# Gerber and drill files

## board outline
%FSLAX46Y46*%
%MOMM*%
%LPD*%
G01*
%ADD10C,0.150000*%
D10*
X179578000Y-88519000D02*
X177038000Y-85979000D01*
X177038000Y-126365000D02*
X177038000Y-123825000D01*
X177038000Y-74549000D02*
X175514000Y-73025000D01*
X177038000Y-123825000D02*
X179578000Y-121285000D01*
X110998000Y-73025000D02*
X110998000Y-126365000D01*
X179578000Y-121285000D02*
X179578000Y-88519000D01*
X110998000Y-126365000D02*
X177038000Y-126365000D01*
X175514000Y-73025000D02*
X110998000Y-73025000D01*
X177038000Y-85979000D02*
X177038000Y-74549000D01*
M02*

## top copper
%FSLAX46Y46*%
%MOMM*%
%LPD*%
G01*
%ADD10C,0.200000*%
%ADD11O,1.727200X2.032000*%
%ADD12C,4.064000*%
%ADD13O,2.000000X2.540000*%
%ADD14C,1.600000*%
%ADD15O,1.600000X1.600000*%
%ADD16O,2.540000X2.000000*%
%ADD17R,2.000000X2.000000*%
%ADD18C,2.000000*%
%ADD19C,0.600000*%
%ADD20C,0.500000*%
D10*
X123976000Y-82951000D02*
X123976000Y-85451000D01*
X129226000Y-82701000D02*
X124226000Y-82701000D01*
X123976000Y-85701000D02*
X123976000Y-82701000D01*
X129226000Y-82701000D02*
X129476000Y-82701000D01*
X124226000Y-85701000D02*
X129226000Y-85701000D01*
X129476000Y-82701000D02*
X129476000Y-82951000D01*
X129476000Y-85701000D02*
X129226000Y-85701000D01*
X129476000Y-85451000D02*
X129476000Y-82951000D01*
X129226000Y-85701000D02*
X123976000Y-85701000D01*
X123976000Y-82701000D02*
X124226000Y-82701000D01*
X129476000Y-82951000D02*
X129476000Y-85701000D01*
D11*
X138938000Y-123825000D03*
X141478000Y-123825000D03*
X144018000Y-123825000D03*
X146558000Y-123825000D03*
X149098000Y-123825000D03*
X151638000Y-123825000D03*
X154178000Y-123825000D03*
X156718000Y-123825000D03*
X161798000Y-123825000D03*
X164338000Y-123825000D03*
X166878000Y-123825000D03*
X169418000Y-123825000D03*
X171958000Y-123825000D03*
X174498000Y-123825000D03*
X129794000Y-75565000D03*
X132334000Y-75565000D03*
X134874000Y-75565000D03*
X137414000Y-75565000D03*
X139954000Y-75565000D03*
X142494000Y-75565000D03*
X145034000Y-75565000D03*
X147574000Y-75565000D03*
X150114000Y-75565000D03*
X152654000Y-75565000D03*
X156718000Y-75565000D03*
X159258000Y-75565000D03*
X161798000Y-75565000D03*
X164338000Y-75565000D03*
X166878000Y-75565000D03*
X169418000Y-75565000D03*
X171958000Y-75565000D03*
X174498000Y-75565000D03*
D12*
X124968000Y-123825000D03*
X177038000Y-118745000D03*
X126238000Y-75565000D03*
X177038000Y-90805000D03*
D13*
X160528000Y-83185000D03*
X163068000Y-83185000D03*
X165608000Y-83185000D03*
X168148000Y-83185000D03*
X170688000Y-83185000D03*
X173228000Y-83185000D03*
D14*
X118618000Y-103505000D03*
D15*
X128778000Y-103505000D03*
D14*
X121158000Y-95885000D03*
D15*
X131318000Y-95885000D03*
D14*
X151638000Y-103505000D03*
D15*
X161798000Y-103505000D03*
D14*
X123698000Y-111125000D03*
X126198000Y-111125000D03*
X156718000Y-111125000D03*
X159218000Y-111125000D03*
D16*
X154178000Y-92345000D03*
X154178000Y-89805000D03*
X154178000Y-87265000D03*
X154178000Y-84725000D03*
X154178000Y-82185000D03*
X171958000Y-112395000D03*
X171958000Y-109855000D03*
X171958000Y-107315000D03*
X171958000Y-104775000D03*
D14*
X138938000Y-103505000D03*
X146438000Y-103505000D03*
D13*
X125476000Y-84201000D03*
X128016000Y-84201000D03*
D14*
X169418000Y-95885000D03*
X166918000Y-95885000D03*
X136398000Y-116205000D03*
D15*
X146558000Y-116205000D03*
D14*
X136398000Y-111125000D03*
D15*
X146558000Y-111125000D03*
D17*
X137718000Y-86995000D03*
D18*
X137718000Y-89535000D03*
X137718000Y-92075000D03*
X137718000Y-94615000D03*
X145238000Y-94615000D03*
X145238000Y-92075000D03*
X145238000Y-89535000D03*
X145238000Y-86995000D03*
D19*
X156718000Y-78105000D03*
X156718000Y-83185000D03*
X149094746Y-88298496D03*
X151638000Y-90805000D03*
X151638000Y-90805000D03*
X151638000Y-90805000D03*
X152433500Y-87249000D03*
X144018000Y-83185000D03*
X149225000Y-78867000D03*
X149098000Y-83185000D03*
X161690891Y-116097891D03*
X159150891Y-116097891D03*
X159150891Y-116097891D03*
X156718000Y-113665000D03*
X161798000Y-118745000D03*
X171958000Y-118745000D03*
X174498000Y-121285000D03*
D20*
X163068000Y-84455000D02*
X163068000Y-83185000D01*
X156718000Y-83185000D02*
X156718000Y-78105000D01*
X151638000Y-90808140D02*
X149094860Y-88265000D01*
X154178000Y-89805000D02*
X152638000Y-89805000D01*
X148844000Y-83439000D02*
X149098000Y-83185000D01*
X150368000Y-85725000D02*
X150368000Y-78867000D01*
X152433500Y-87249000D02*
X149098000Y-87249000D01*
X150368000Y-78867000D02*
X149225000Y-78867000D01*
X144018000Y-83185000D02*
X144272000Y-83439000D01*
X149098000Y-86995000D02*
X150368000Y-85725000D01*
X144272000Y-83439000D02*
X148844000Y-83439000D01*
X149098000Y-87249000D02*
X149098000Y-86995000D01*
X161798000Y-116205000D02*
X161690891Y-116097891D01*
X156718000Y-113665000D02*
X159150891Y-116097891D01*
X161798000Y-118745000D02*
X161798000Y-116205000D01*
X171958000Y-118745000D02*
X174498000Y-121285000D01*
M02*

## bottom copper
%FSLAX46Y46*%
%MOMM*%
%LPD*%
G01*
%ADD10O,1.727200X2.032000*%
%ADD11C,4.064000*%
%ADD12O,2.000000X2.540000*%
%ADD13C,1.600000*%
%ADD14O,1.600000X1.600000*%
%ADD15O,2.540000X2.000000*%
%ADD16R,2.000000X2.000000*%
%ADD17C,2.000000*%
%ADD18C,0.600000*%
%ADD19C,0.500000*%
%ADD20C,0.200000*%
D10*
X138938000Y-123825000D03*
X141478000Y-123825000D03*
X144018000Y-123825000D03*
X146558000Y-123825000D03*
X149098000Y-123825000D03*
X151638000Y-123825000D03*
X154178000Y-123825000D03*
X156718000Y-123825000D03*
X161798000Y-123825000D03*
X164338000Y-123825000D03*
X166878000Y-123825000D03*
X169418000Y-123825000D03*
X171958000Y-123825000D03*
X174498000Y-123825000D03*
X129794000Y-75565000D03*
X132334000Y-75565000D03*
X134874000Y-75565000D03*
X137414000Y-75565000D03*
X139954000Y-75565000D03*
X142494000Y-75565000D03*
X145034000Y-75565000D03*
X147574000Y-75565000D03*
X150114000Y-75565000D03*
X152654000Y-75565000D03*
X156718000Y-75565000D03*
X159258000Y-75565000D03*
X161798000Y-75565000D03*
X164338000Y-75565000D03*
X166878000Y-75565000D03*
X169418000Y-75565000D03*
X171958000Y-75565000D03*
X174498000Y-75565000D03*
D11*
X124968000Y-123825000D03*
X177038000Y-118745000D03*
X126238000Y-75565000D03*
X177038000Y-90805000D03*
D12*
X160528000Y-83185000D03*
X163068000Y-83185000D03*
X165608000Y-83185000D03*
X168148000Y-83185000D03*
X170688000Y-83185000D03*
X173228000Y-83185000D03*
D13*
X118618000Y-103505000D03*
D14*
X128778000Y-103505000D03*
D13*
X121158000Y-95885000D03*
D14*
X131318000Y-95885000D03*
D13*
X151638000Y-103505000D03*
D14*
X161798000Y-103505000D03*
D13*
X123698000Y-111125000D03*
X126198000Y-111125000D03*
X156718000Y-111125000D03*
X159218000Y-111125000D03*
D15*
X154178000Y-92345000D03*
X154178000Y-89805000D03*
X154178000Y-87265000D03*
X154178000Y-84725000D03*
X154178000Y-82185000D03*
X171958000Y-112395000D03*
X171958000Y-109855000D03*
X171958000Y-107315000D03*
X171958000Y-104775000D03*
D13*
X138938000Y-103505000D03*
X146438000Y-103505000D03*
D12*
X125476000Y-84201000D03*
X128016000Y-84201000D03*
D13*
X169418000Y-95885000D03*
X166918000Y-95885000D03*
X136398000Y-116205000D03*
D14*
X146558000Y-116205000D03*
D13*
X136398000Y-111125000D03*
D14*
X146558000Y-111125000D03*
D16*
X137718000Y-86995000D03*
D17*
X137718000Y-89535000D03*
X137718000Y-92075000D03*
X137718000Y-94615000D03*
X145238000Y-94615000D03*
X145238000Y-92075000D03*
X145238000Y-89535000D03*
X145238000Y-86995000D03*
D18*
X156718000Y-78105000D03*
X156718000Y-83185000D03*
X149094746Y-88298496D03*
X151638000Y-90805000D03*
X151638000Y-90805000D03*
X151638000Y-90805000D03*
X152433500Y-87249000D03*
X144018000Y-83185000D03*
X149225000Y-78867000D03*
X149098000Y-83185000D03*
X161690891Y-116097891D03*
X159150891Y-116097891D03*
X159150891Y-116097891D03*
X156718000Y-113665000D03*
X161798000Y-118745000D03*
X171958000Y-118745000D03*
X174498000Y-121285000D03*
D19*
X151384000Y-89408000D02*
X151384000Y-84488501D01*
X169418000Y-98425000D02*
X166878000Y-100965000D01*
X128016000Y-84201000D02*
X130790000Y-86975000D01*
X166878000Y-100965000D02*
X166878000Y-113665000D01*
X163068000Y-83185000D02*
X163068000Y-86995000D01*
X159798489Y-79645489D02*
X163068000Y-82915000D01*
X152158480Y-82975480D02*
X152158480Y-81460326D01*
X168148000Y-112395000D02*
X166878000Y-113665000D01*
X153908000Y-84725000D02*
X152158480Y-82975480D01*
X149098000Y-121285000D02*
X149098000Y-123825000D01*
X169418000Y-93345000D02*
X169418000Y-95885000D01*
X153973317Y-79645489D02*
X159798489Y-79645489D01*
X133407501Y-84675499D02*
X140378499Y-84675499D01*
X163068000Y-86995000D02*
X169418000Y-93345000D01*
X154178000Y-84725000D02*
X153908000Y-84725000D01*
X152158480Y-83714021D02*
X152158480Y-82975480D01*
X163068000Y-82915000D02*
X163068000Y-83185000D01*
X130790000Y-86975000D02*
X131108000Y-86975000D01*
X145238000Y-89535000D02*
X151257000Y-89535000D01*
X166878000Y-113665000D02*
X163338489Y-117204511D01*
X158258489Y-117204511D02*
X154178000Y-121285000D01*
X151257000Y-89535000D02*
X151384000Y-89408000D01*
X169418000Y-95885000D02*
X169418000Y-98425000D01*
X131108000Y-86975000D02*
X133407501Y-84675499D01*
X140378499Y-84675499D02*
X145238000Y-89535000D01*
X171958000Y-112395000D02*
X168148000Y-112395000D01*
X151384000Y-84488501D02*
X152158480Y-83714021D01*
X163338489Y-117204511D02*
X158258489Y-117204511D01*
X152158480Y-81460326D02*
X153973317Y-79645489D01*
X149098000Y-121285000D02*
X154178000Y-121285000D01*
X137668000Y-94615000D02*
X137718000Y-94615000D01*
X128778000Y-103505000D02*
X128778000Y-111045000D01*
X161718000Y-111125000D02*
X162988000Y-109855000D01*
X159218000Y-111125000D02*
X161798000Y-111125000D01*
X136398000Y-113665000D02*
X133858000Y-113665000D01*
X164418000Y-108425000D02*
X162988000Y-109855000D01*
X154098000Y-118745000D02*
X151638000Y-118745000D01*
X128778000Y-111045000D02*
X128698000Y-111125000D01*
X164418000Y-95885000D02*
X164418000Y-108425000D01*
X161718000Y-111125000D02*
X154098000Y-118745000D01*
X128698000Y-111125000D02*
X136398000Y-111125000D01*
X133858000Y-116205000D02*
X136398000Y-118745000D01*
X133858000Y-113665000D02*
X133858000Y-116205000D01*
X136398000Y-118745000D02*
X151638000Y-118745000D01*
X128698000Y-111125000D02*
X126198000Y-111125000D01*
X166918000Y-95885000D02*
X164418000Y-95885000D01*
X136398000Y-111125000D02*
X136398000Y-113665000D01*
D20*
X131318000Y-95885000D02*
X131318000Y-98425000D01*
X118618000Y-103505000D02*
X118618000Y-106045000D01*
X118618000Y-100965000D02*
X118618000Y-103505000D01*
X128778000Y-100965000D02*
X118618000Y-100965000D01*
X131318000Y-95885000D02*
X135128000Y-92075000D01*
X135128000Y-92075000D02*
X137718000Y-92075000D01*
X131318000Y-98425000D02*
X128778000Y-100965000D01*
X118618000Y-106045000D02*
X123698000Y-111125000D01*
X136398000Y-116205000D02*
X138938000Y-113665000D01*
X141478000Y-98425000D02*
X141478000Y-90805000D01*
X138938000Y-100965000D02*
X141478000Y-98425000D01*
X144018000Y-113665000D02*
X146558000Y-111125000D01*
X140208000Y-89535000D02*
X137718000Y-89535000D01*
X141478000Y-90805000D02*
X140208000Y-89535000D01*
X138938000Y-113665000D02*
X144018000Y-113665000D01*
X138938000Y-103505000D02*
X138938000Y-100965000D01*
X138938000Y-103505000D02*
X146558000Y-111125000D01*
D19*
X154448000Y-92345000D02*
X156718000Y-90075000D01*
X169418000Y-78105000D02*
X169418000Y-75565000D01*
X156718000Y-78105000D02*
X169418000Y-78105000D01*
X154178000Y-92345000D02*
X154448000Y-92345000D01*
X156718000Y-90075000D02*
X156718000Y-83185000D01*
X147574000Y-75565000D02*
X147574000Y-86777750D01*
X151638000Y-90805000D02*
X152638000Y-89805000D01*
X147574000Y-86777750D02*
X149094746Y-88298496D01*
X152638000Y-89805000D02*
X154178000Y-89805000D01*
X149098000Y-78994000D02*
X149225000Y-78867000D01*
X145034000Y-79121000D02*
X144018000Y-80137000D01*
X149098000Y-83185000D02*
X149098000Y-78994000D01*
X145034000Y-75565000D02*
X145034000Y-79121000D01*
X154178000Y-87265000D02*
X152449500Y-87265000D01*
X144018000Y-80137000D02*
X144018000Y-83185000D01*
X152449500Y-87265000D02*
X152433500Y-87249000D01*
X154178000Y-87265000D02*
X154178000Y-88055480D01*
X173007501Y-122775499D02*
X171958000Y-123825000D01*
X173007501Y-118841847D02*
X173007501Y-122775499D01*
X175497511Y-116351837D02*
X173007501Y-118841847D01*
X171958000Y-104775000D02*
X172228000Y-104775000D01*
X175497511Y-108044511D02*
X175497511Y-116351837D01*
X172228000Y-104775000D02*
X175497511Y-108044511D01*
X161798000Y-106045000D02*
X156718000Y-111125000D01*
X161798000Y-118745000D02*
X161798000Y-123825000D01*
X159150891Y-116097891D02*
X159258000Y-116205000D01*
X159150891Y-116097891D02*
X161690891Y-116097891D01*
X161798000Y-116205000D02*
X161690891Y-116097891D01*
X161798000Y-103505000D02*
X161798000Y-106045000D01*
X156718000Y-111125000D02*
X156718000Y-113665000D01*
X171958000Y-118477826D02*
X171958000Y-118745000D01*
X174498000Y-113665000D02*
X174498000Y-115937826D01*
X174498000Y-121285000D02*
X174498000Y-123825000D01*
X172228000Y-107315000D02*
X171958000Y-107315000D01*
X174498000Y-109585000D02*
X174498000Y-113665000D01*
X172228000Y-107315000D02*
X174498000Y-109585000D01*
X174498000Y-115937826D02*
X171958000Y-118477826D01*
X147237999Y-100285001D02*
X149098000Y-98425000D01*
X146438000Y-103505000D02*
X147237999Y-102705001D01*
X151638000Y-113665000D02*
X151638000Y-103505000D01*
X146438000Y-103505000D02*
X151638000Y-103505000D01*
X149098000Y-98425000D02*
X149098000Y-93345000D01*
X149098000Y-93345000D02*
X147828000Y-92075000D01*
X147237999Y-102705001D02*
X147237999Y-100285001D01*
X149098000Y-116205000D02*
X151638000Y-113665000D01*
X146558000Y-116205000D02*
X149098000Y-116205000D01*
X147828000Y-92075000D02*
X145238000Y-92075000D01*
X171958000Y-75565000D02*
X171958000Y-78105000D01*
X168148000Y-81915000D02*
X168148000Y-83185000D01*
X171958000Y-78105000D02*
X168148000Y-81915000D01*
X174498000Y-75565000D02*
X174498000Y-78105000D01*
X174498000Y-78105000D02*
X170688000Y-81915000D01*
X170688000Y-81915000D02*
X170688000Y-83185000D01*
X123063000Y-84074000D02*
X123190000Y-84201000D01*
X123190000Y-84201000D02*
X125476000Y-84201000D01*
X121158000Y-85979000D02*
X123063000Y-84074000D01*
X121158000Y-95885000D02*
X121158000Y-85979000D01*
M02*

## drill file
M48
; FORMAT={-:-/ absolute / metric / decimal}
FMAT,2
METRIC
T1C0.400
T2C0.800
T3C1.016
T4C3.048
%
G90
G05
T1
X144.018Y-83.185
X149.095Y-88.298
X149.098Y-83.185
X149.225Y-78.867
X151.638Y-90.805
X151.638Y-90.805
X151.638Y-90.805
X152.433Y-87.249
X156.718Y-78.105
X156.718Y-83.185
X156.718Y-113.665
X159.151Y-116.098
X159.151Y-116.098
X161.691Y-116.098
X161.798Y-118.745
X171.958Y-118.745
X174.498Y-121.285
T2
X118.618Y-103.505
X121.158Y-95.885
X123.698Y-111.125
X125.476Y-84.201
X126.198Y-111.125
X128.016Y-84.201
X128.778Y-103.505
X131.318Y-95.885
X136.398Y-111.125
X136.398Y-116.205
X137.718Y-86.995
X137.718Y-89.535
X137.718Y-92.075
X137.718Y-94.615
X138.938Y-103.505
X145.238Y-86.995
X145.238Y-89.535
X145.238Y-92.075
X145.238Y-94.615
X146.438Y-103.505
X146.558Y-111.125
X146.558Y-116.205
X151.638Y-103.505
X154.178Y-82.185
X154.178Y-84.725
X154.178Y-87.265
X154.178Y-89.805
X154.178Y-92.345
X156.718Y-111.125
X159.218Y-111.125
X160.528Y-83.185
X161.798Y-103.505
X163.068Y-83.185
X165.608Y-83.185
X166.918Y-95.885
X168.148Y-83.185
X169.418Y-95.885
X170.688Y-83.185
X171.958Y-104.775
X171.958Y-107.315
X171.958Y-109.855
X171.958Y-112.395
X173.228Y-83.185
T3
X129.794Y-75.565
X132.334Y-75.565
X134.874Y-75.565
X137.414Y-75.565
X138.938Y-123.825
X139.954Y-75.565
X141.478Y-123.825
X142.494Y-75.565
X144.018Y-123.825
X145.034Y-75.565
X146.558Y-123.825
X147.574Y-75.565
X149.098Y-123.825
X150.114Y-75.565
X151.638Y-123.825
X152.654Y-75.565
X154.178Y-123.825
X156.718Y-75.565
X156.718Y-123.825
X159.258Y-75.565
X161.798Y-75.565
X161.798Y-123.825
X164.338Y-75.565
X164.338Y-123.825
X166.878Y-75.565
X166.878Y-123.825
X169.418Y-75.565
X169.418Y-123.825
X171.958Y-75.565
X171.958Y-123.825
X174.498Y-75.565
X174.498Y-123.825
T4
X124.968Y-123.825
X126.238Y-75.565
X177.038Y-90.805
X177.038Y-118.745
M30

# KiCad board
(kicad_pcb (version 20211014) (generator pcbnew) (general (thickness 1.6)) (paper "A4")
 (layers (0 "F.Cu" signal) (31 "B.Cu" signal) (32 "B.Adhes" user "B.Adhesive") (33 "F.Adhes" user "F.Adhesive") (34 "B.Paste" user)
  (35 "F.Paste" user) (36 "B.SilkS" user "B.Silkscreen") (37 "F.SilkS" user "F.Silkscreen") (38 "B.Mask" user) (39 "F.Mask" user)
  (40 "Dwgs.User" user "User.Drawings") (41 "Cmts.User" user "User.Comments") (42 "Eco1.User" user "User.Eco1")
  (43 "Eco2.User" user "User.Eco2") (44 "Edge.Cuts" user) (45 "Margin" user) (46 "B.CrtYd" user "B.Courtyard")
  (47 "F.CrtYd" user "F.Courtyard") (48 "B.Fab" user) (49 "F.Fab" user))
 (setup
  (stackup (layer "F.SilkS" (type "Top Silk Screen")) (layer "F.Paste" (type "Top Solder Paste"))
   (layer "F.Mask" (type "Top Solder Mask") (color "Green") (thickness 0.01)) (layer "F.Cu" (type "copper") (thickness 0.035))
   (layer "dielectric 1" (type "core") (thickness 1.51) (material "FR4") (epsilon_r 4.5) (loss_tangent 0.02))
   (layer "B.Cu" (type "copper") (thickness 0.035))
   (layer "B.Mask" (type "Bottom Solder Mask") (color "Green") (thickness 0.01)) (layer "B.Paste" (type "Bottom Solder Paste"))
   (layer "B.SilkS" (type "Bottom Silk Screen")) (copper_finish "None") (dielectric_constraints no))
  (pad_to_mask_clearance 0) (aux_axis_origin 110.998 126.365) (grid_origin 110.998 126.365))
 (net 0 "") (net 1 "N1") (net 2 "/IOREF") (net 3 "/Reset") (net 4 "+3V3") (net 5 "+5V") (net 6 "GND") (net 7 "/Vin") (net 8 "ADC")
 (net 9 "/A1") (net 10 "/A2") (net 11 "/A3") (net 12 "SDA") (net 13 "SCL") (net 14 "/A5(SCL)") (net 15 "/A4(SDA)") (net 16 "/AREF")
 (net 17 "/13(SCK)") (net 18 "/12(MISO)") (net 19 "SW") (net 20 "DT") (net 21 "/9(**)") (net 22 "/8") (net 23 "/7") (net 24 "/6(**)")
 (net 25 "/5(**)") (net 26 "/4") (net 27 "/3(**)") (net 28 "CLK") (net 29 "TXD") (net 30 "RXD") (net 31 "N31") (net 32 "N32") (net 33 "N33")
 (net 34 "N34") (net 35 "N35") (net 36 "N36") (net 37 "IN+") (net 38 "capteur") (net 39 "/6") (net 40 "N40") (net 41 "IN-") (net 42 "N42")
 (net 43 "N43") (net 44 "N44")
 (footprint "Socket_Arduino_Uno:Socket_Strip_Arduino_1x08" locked (layer "F.Cu") (at 138.938 123.825)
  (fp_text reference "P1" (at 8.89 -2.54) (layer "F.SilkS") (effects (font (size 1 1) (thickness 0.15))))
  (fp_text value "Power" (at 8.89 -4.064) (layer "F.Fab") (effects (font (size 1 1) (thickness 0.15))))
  (pad "1" thru_hole oval locked (at 0 0) (size 1.7272 2.032) (drill 1.016) (layers *.Cu *.Mask "F.SilkS") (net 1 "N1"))
  (pad "2" thru_hole oval locked (at 2.54 0) (size 1.7272 2.032) (drill 1.016) (layers *.Cu *.Mask "F.SilkS") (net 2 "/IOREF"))
  (pad "3" thru_hole oval locked (at 5.08 0) (size 1.7272 2.032) (drill 1.016) (layers *.Cu *.Mask "F.SilkS") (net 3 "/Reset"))
  (pad "4" thru_hole oval locked (at 7.62 0) (size 1.7272 2.032) (drill 1.016) (layers *.Cu *.Mask "F.SilkS") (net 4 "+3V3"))
  (pad "5" thru_hole oval locked (at 10.16 0) (size 1.7272 2.032) (drill 1.016) (layers *.Cu *.Mask "F.SilkS") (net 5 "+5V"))
  (pad "6" thru_hole oval locked (at 12.7 0) (size 1.7272 2.032) (drill 1.016) (layers *.Cu *.Mask "F.SilkS") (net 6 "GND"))
  (pad "7" thru_hole oval locked (at 15.24 0) (size 1.7272 2.032) (drill 1.016) (layers *.Cu *.Mask "F.SilkS") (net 6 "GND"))
  (pad "8" thru_hole oval locked (at 17.78 0) (size 1.7272 2.032) (drill 1.016) (layers *.Cu *.Mask "F.SilkS") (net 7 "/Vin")))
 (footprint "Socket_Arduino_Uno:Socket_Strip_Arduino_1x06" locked (layer "F.Cu") (at 161.798 123.825)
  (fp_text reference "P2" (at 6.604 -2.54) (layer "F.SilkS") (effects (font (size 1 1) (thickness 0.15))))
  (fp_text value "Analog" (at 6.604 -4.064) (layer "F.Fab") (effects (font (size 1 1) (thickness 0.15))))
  (pad "1" thru_hole oval locked (at 0 0) (size 1.7272 2.032) (drill 1.016) (layers *.Cu *.Mask "F.SilkS") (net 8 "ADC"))
  (pad "2" thru_hole oval locked (at 2.54 0) (size 1.7272 2.032) (drill 1.016) (layers *.Cu *.Mask "F.SilkS") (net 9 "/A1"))
  (pad "3" thru_hole oval locked (at 5.08 0) (size 1.7272 2.032) (drill 1.016) (layers *.Cu *.Mask "F.SilkS") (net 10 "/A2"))
  (pad "4" thru_hole oval locked (at 7.62 0) (size 1.7272 2.032) (drill 1.016) (layers *.Cu *.Mask "F.SilkS") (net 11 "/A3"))
  (pad "5" thru_hole oval locked (at 10.16 0) (size 1.7272 2.032) (drill 1.016) (layers *.Cu *.Mask "F.SilkS") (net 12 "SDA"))
  (pad "6" thru_hole oval locked (at 12.7 0) (size 1.7272 2.032) (drill 1.016) (layers *.Cu *.Mask "F.SilkS") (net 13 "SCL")))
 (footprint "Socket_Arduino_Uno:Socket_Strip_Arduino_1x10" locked (layer "F.Cu") (at 129.794 75.565)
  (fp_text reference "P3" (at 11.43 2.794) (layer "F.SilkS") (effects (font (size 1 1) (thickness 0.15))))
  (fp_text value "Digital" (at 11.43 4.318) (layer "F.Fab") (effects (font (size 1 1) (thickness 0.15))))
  (pad "1" thru_hole oval locked (at 0 0) (size 1.7272 2.032) (drill 1.016) (layers *.Cu *.Mask "F.SilkS") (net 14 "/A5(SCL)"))
  (pad "2" thru_hole oval locked (at 2.54 0) (size 1.7272 2.032) (drill 1.016) (layers *.Cu *.Mask "F.SilkS") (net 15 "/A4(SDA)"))
  (pad "3" thru_hole oval locked (at 5.08 0) (size 1.7272 2.032) (drill 1.016) (layers *.Cu *.Mask "F.SilkS") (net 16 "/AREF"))
  (pad "4" thru_hole oval locked (at 7.62 0) (size 1.7272 2.032) (drill 1.016) (layers *.Cu *.Mask "F.SilkS") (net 6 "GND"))
  (pad "5" thru_hole oval locked (at 10.16 0) (size 1.7272 2.032) (drill 1.016) (layers *.Cu *.Mask "F.SilkS") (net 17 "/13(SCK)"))
  (pad "6" thru_hole oval locked (at 12.7 0) (size 1.7272 2.032) (drill 1.016) (layers *.Cu *.Mask "F.SilkS") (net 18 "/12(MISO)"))
  (pad "7" thru_hole oval locked (at 15.24 0) (size 1.7272 2.032) (drill 1.016) (layers *.Cu *.Mask "F.SilkS") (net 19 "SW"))
  (pad "8" thru_hole oval locked (at 17.78 0) (size 1.7272 2.032) (drill 1.016) (layers *.Cu *.Mask "F.SilkS") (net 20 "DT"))
  (pad "9" thru_hole oval locked (at 20.32 0) (size 1.7272 2.032) (drill 1.016) (layers *.Cu *.Mask "F.SilkS") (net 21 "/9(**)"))
  (pad "10" thru_hole oval locked (at 22.86 0) (size 1.7272 2.032) (drill 1.016) (layers *.Cu *.Mask "F.SilkS") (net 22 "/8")))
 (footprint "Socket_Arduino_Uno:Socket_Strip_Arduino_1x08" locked (layer "F.Cu") (at 156.718 75.565)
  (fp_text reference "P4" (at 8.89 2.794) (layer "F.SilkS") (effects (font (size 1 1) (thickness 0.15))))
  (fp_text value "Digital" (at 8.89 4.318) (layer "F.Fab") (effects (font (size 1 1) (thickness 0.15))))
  (pad "1" thru_hole oval locked (at 0 0) (size 1.7272 2.032) (drill 1.016) (layers *.Cu *.Mask "F.SilkS") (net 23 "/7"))
  (pad "2" thru_hole oval locked (at 2.54 0) (size 1.7272 2.032) (drill 1.016) (layers *.Cu *.Mask "F.SilkS") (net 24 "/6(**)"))
  (pad "3" thru_hole oval locked (at 5.08 0) (size 1.7272 2.032) (drill 1.016) (layers *.Cu *.Mask "F.SilkS") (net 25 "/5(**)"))
  (pad "4" thru_hole oval locked (at 7.62 0) (size 1.7272 2.032) (drill 1.016) (layers *.Cu *.Mask "F.SilkS") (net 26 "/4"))
  (pad "5" thru_hole oval locked (at 10.16 0) (size 1.7272 2.032) (drill 1.016) (layers *.Cu *.Mask "F.SilkS") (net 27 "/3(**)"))
  (pad "6" thru_hole oval locked (at 12.7 0) (size 1.7272 2.032) (drill 1.016) (layers *.Cu *.Mask "F.SilkS") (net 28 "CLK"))
  (pad "7" thru_hole oval locked (at 15.24 0) (size 1.7272 2.032) (drill 1.016) (layers *.Cu *.Mask "F.SilkS") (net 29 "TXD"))
  (pad "8" thru_hole oval locked (at 17.78 0) (size 1.7272 2.032) (drill 1.016) (layers *.Cu *.Mask "F.SilkS") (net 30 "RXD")))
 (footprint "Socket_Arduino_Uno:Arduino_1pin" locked (layer "F.Cu") (at 124.968 123.825)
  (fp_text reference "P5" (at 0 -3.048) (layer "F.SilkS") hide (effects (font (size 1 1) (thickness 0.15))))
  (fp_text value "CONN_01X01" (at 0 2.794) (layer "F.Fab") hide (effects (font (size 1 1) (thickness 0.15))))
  (pad "1" thru_hole circle locked (at 0 0) (size 4.064 4.064) (drill 3.048) (layers *.Cu *.Mask "F.SilkS") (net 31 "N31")))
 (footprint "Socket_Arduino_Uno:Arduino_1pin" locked (layer "F.Cu") (at 177.038 118.745)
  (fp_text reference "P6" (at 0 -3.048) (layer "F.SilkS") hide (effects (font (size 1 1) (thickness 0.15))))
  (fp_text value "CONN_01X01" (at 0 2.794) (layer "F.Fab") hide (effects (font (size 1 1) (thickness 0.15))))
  (pad "1" thru_hole circle locked (at 0 0) (size 4.064 4.064) (drill 3.048) (layers *.Cu *.Mask "F.SilkS") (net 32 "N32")))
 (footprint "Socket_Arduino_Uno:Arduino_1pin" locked (layer "F.Cu") (at 126.238 75.565)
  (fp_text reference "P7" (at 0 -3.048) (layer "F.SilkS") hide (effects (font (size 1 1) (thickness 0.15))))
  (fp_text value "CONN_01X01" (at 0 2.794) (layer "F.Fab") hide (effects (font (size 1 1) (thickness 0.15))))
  (pad "1" thru_hole circle locked (at 0 0) (size 4.064 4.064) (drill 3.048) (layers *.Cu *.Mask "F.SilkS") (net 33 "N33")))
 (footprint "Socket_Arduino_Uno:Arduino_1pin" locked (layer "F.Cu") (at 177.038 90.805)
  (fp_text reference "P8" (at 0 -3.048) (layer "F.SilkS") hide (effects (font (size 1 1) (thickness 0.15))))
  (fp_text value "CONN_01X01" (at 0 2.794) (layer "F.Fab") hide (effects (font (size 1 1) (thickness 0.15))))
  (pad "1" thru_hole circle locked (at 0 0) (size 4.064 4.064) (drill 3.048) (layers *.Cu *.Mask "F.SilkS") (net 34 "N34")))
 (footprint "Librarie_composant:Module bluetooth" (layer "F.Cu") (at 166.878 83.185)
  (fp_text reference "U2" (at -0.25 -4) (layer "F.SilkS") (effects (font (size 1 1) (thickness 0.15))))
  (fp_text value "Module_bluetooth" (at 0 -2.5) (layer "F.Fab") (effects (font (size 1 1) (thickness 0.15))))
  (pad "1" thru_hole oval (at -6.35 0) (size 2 2.54) (drill 0.8) (layers *.Cu *.Mask) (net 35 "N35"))
  (pad "2" thru_hole oval (at -3.81 0) (size 2 2.54) (drill 0.8) (layers *.Cu *.Mask) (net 5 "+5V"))
  (pad "3" thru_hole oval (at -1.27 0) (size 2 2.54) (drill 0.8) (layers *.Cu *.Mask) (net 6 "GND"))
  (pad "4" thru_hole oval (at 1.27 0) (size 2 2.54) (drill 0.8) (layers *.Cu *.Mask) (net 29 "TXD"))
  (pad "5" thru_hole oval (at 3.81 0) (size 2 2.54) (drill 0.8) (layers *.Cu *.Mask) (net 30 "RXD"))
  (pad "6" thru_hole oval (at 6.35 0) (size 2 2.54) (drill 0.8) (layers *.Cu *.Mask) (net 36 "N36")))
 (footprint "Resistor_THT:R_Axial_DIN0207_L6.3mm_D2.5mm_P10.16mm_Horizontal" (layer "F.Cu") (at 118.618 103.505)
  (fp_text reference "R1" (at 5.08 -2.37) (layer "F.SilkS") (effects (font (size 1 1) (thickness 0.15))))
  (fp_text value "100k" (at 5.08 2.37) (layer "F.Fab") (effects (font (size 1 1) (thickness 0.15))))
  (pad "1" thru_hole circle (at 0 0) (size 1.6 1.6) (drill 0.8) (layers *.Cu *.Mask) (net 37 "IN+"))
  (pad "2" thru_hole oval (at 10.16 0) (size 1.6 1.6) (drill 0.8) (layers *.Cu *.Mask) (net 6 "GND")))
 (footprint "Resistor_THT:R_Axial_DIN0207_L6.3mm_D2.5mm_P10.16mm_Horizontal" (layer "F.Cu") (at 121.158 95.885)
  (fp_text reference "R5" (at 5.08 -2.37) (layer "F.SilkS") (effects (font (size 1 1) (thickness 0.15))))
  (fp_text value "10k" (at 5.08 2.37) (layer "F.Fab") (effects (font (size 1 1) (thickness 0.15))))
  (pad "1" thru_hole circle (at 0 0) (size 1.6 1.6) (drill 0.8) (layers *.Cu *.Mask) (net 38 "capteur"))
  (pad "2" thru_hole oval (at 10.16 0) (size 1.6 1.6) (drill 0.8) (layers *.Cu *.Mask) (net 37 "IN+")))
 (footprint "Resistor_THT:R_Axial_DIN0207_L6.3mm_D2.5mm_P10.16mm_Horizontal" (layer "F.Cu") (at 151.638 103.505)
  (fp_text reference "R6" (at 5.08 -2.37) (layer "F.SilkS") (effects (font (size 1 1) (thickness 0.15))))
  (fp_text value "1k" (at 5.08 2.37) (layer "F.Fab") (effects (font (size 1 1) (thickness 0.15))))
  (pad "1" thru_hole circle (at 0 0) (size 1.6 1.6) (drill 0.8) (layers *.Cu *.Mask) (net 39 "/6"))
  (pad "2" thru_hole oval (at 10.16 0) (size 1.6 1.6) (drill 0.8) (layers *.Cu *.Mask) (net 8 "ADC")))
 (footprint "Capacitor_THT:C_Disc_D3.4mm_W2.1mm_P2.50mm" (layer "F.Cu") (at 123.698 111.125)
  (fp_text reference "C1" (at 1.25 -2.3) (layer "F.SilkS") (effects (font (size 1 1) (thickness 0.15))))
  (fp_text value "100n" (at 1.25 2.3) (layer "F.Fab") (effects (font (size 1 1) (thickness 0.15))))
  (pad "1" thru_hole circle (at 0 0) (size 1.6 1.6) (drill 0.8) (layers *.Cu *.Mask) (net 37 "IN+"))
  (pad "2" thru_hole circle (at 2.5 0) (size 1.6 1.6) (drill 0.8) (layers *.Cu *.Mask) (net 6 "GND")))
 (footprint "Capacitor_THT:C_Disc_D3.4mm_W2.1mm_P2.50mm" (layer "F.Cu") (at 156.718 111.125)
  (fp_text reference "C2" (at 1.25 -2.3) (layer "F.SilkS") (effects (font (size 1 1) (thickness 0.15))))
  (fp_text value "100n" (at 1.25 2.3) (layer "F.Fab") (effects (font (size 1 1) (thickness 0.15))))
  (pad "1" thru_hole circle (at 0 0) (size 1.6 1.6) (drill 0.8) (layers *.Cu *.Mask) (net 8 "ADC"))
  (pad "2" thru_hole circle (at 2.5 0) (size 1.6 1.6) (drill 0.8) (layers *.Cu *.Mask) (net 6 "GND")))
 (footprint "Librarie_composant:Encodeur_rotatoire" (layer "F.Cu") (at 154.178 88.265 90)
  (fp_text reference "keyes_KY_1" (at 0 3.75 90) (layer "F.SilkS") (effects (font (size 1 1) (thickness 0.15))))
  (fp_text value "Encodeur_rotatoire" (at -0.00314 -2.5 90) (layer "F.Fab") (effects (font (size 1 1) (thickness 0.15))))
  (pad "1" thru_hole oval (at -4.08 0 90) (size 2 2.54) (drill 0.8) (layers *.Cu *.Mask) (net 28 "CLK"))
  (pad "2" thru_hole oval (at -1.54 0 90) (size 2 2.54) (drill 0.8) (layers *.Cu *.Mask) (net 20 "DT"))
  (pad "3" thru_hole oval (at 1 0 90) (size 2 2.54) (drill 0.8) (layers *.Cu *.Mask "Eco1.User") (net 19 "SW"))
  (pad "4" thru_hole oval (at 3.54 0 90) (size 2 2.54) (drill 0.8) (layers *.Cu *.Mask) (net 5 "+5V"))
  (pad "5" thru_hole oval (at 6.08 0 90) (size 2 2.54) (drill 0.8) (layers *.Cu *.Mask) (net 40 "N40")))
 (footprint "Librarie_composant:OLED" (layer "F.Cu") (at 171.958 108.585 90)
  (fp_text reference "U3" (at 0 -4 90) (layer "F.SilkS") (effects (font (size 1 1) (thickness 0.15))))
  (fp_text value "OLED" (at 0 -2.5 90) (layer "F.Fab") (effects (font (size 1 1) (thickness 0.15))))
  (pad "1" thru_hole oval (at -3.81 0 90) (size 2 2.54) (drill 0.8) (layers *.Cu *.Mask) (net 5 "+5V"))
  (pad "2" thru_hole oval (at -1.27 0 90) (size 2 2.54) (drill 0.8) (layers *.Cu *.Mask) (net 6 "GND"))
  (pad "3" thru_hole oval (at 1.27 0 90) (size 2 2.54) (drill 0.8) (layers *.Cu *.Mask) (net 13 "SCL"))
  (pad "4" thru_hole oval (at 3.81 0 90) (size 2 2.54) (drill 0.8) (layers *.Cu *.Mask) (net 12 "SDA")))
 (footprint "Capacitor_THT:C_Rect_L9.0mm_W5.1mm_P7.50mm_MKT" (layer "F.Cu") (at 138.938 103.505)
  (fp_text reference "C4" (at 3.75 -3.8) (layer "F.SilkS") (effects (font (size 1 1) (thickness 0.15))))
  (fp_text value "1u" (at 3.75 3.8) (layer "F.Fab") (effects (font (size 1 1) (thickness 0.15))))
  (pad "1" thru_hole circle (at 0 0) (size 1.6 1.6) (drill 0.8) (layers *.Cu *.Mask) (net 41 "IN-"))
  (pad "2" thru_hole circle (at 7.5 0) (size 1.6 1.6) (drill 0.8) (layers *.Cu *.Mask) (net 39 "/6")))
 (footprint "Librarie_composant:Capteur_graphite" (layer "F.Cu") (at 126.476 84.201)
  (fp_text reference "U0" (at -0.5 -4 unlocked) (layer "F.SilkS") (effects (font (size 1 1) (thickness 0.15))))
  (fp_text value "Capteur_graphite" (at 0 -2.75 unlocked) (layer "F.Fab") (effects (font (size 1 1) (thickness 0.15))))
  (fp_line (start -2.5 -1.25) (end -2.5 1.25) (layer "F.Cu") (width 0.2))
  (fp_line (start 2.75 -1.5) (end -2.25 -1.5) (layer "F.Cu") (width 0.2))
  (fp_line (start -2.5 1.5) (end -2.5 -1.5) (layer "F.Cu") (width 0.2))
  (fp_line (start 2.75 -1.5) (end 3 -1.5) (layer "F.Cu") (width 0.2))
  (fp_line (start -2.25 1.5) (end 2.75 1.5) (layer "F.Cu") (width 0.2))
  (fp_line (start 3 -1.5) (end 3 -1.25) (layer "F.Cu") (width 0.2))
  (fp_line (start 3 1.5) (end 2.75 1.5) (layer "F.Cu") (width 0.2))
  (fp_line (start 3 1.25) (end 3 -1.25) (layer "F.Cu") (width 0.2))
  (fp_line (start 2.75 1.5) (end -2.5 1.5) (layer "F.Cu") (width 0.2))
  (fp_line (start -2.5 -1.5) (end -2.25 -1.5) (layer "F.Cu") (width 0.2))
  (fp_line (start 3 -1.25) (end 3 1.5) (layer "F.Cu") (width 0.2))
  (pad "1" thru_hole oval (at -1 0) (size 2 2.54) (drill 0.8) (layers *.Cu *.Mask) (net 38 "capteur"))
  (pad "2" thru_hole oval (at 1.54 0) (size 2 2.54) (drill 0.8) (layers *.Cu *.Mask) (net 5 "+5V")))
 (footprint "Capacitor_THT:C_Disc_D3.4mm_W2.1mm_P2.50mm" (layer "F.Cu") (at 169.418 95.885 180)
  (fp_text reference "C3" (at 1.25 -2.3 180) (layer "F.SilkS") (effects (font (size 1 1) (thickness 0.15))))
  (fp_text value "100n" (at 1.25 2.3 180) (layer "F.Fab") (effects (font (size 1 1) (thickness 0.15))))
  (pad "1" thru_hole circle (at 0 0 180) (size 1.6 1.6) (drill 0.8) (layers *.Cu *.Mask) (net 5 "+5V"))
  (pad "2" thru_hole circle (at 2.5 0 180) (size 1.6 1.6) (drill 0.8) (layers *.Cu *.Mask) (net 6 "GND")))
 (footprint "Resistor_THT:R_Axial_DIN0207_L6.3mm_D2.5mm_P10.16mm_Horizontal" (layer "F.Cu") (at 136.398 116.205)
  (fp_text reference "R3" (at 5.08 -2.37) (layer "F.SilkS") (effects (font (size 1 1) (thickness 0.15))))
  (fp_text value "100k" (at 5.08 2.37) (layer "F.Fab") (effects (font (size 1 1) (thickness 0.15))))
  (pad "1" thru_hole circle (at 0 0) (size 1.6 1.6) (drill 0.8) (layers *.Cu *.Mask) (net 41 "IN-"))
  (pad "2" thru_hole oval (at 10.16 0) (size 1.6 1.6) (drill 0.8) (layers *.Cu *.Mask) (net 39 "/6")))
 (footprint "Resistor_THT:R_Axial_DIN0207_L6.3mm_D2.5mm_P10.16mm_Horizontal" (layer "F.Cu") (at 136.398 111.125)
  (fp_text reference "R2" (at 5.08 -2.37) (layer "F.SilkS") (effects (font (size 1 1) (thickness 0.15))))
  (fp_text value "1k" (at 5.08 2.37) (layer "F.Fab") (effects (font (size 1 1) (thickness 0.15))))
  (pad "1" thru_hole circle (at 0 0) (size 1.6 1.6) (drill 0.8) (layers *.Cu *.Mask) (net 6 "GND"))
  (pad "2" thru_hole oval (at 10.16 0) (size 1.6 1.6) (drill 0.8) (layers *.Cu *.Mask) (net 41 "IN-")))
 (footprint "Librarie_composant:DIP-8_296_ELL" (layer "F.Cu") (at 141.478 90.805 -90)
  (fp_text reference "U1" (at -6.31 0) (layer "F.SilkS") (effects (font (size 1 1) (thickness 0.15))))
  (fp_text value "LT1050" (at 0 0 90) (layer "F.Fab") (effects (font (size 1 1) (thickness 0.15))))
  (pad "1" thru_hole rect (at -3.81 3.76 270) (size 2 2) (drill 0.8) (layers *.Cu *.Mask) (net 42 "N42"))
  (pad "2" thru_hole circle (at -1.27 3.76 270) (size 2 2) (drill 0.8) (layers *.Cu *.Mask) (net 41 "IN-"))
  (pad "3" thru_hole circle (at 1.27 3.76 270) (size 2 2) (drill 0.8) (layers *.Cu *.Mask) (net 37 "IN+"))
  (pad "4" thru_hole circle (at 3.81 3.76 270) (size 2 2) (drill 0.8) (layers *.Cu *.Mask) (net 6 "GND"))
  (pad "5" thru_hole circle (at 3.81 -3.76 270) (size 2 2) (drill 0.8) (layers *.Cu *.Mask) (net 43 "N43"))
  (pad "6" thru_hole circle (at 1.27 -3.76 270) (size 2 2) (drill 0.8) (layers *.Cu *.Mask) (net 39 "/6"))
  (pad "7" thru_hole circle (at -1.27 -3.76 270) (size 2 2) (drill 0.8) (layers *.Cu *.Mask) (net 5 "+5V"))
  (pad "8" thru_hole circle (at -3.81 -3.76 270) (size 2 2) (drill 0.8) (layers *.Cu *.Mask) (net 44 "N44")))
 (gr_line (start 179.578 88.519) (end 177.038 85.979) (layer "Edge.Cuts") (width 0.15))
 (gr_line (start 177.038 126.365) (end 177.038 123.825) (layer "Edge.Cuts") (width 0.15))
 (gr_line (start 177.038 74.549) (end 175.514 73.025) (layer "Edge.Cuts") (width 0.15))
 (gr_line (start 177.038 123.825) (end 179.578 121.285) (layer "Edge.Cuts") (width 0.15))
 (gr_line (start 110.998 73.025) (end 110.998 126.365) (layer "Edge.Cuts") (width 0.15))
 (gr_line (start 179.578 121.285) (end 179.578 88.519) (layer "Edge.Cuts") (width 0.15))
 (gr_line (start 110.998 126.365) (end 177.038 126.365) (layer "Edge.Cuts") (width 0.15))
 (gr_line (start 175.514 73.025) (end 110.998 73.025) (layer "Edge.Cuts") (width 0.15))
 (gr_line (start 177.038 85.979) (end 177.038 74.549) (layer "Edge.Cuts") (width 0.15))
 (segment (start 163.068 84.455) (end 163.068 83.185) (width 0.5) (layer "F.Cu") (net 5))
 (segment (start 151.384 89.408) (end 151.384 84.488501) (width 0.5) (layer "B.Cu") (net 5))
 (segment (start 169.418 98.425) (end 166.878 100.965) (width 0.5) (layer "B.Cu") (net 5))
 (segment (start 128.016 84.201) (end 130.79 86.975) (width 0.5) (layer "B.Cu") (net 5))
 (segment (start 166.878 100.965) (end 166.878 113.665) (width 0.5) (layer "B.Cu") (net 5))
 (segment (start 163.068 83.185) (end 163.068 86.995) (width 0.5) (layer "B.Cu") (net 5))
 (segment (start 159.798489 79.645489) (end 163.068 82.915) (width 0.5) (layer "B.Cu") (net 5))
 (segment (start 152.15848 82.97548) (end 152.15848 81.460326) (width 0.5) (layer "B.Cu") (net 5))
 (segment (start 168.148 112.395) (end 166.878 113.665) (width 0.5) (layer "B.Cu") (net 5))
 (segment (start 153.908 84.725) (end 152.15848 82.97548) (width 0.5) (layer "B.Cu") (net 5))
 (segment (start 149.098 121.285) (end 149.098 123.825) (width 0.5) (layer "B.Cu") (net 5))
 (segment (start 169.418 93.345) (end 169.418 95.885) (width 0.5) (layer "B.Cu") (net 5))
 (segment (start 153.973317 79.645489) (end 159.798489 79.645489) (width 0.5) (layer "B.Cu") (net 5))
 (segment (start 133.407501 84.675499) (end 140.378499 84.675499) (width 0.5) (layer "B.Cu") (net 5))
 (segment (start 163.068 86.995) (end 169.418 93.345) (width 0.5) (layer "B.Cu") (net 5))
 (segment (start 154.178 84.725) (end 153.908 84.725) (width 0.5) (layer "B.Cu") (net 5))
 (segment (start 152.15848 83.714021) (end 152.15848 82.97548) (width 0.5) (layer "B.Cu") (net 5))
 (segment (start 163.068 82.915) (end 163.068 83.185) (width 0.5) (layer "B.Cu") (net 5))
 (segment (start 130.79 86.975) (end 131.108 86.975) (width 0.5) (layer "B.Cu") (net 5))
 (segment (start 145.238 89.535) (end 151.257 89.535) (width 0.5) (layer "B.Cu") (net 5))
 (segment (start 166.878 113.665) (end 163.338489 117.204511) (width 0.5) (layer "B.Cu") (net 5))
 (segment (start 158.258489 117.204511) (end 154.178 121.285) (width 0.5) (layer "B.Cu") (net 5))
 (segment (start 151.257 89.535) (end 151.384 89.408) (width 0.5) (layer "B.Cu") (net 5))
 (segment (start 169.418 95.885) (end 169.418 98.425) (width 0.5) (layer "B.Cu") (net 5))
 (segment (start 131.108 86.975) (end 133.407501 84.675499) (width 0.5) (layer "B.Cu") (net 5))
 (segment (start 140.378499 84.675499) (end 145.238 89.535) (width 0.5) (layer "B.Cu") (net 5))
 (segment (start 171.958 112.395) (end 168.148 112.395) (width 0.5) (layer "B.Cu") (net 5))
 (segment (start 151.384 84.488501) (end 152.15848 83.714021) (width 0.5) (layer "B.Cu") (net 5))
 (segment (start 163.338489 117.204511) (end 158.258489 117.204511) (width 0.5) (layer "B.Cu") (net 5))
 (segment (start 152.15848 81.460326) (end 153.973317 79.645489) (width 0.5) (layer "B.Cu") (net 5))
 (segment (start 149.098 121.285) (end 154.178 121.285) (width 0.5) (layer "B.Cu") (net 5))
 (segment (start 137.668 94.615) (end 137.718 94.615) (width 0.5) (layer "B.Cu") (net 6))
 (segment (start 128.778 103.505) (end 128.778 111.045) (width 0.5) (layer "B.Cu") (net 6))
 (segment (start 161.718 111.125) (end 162.988 109.855) (width 0.5) (layer "B.Cu") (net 6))
 (segment (start 159.218 111.125) (end 161.798 111.125) (width 0.5) (layer "B.Cu") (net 6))
 (segment (start 136.398 113.665) (end 133.858 113.665) (width 0.5) (layer "B.Cu") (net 6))
 (segment (start 164.418 108.425) (end 162.988 109.855) (width 0.5) (layer "B.Cu") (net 6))
 (segment (start 154.098 118.745) (end 151.638 118.745) (width 0.5) (layer "B.Cu") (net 6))
 (segment (start 128.778 111.045) (end 128.698 111.125) (width 0.5) (layer "B.Cu") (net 6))
 (segment (start 164.418 95.885) (end 164.418 108.425) (width 0.5) (layer "B.Cu") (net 6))
 (segment (start 161.718 111.125) (end 154.098 118.745) (width 0.5) (layer "B.Cu") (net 6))
 (segment (start 128.698 111.125) (end 136.398 111.125) (width 0.5) (layer "B.Cu") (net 6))
 (segment (start 133.858 116.205) (end 136.398 118.745) (width 0.5) (layer "B.Cu") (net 6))
 (segment (start 133.858 113.665) (end 133.858 116.205) (width 0.5) (layer "B.Cu") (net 6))
 (segment (start 136.398 118.745) (end 151.638 118.745) (width 0.5) (layer "B.Cu") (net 6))
 (segment (start 128.698 111.125) (end 126.198 111.125) (width 0.5) (layer "B.Cu") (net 6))
 (segment (start 166.918 95.885) (end 164.418 95.885) (width 0.5) (layer "B.Cu") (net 6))
 (segment (start 136.398 111.125) (end 136.398 113.665) (width 0.5) (layer "B.Cu") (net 6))
 (segment (start 131.318 95.885) (end 131.318 98.425) (width 0.2) (layer "B.Cu") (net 37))
 (segment (start 118.618 103.505) (end 118.618 106.045) (width 0.2) (layer "B.Cu") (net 37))
 (segment (start 118.618 100.965) (end 118.618 103.505) (width 0.2) (layer "B.Cu") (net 37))
 (segment (start 128.778 100.965) (end 118.618 100.965) (width 0.2) (layer "B.Cu") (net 37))
 (segment (start 131.318 95.885) (end 135.128 92.075) (width 0.2) (layer "B.Cu") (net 37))
 (segment (start 135.128 92.075) (end 137.718 92.075) (width 0.2) (layer "B.Cu") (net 37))
 (segment (start 131.318 98.425) (end 128.778 100.965) (width 0.2) (layer "B.Cu") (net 37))
 (segment (start 118.618 106.045) (end 123.698 111.125) (width 0.2) (layer "B.Cu") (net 37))
 (segment (start 136.398 116.205) (end 138.938 113.665) (width 0.2) (layer "B.Cu") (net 41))
 (segment (start 141.478 98.425) (end 141.478 90.805) (width 0.2) (layer "B.Cu") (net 41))
 (segment (start 138.938 100.965) (end 141.478 98.425) (width 0.2) (layer "B.Cu") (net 41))
 (segment (start 144.018 113.665) (end 146.558 111.125) (width 0.2) (layer "B.Cu") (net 41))
 (segment (start 140.208 89.535) (end 137.718 89.535) (width 0.2) (layer "B.Cu") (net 41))
 (segment (start 141.478 90.805) (end 140.208 89.535) (width 0.2) (layer "B.Cu") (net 41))
 (segment (start 138.938 113.665) (end 144.018 113.665) (width 0.2) (layer "B.Cu") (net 41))
 (segment (start 138.938 103.505) (end 138.938 100.965) (width 0.2) (layer "B.Cu") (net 41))
 (segment (start 138.938 103.505) (end 146.558 111.125) (width 0.2) (layer "B.Cu") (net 41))
 (segment (start 156.718 83.185) (end 156.718 78.105) (width 0.5) (layer "F.Cu") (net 28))
 (via (at 156.718 78.105) (size 0.6) (drill 0.4) (layers "F.Cu" "B.Cu") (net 28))
 (via (at 156.718 83.185) (size 0.6) (drill 0.4) (layers "F.Cu" "B.Cu") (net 28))
 (segment (start 154.448 92.345) (end 156.718 90.075) (width 0.5) (layer "B.Cu") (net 28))
 (segment (start 169.418 78.105) (end 169.418 75.565) (width 0.5) (layer "B.Cu") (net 28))
 (segment (start 156.718 78.105) (end 169.418 78.105) (width 0.5) (layer "B.Cu") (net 28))
 (segment (start 154.178 92.345) (end 154.448 92.345) (width 0.5) (layer "B.Cu") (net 28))
 (segment (start 156.718 90.075) (end 156.718 83.185) (width 0.5) (layer "B.Cu") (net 28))
 (segment (start 151.638 90.80814) (end 149.09486 88.265) (width 0.5) (layer "F.Cu") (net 20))
 (segment (start 154.178 89.805) (end 152.638 89.805) (width 0.5) (layer "F.Cu") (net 20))
 (via (at 149.094746 88.298496) (size 0.6) (drill 0.4) (layers "F.Cu" "B.Cu") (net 20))
 (via (at 151.638 90.805) (size 0.6) (drill 0.4) (layers "F.Cu" "B.Cu") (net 20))
 (via (at 151.638 90.805) (size 0.6) (drill 0.4) (layers "F.Cu" "B.Cu") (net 20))
 (via (at 151.638 90.805) (size 0.6) (drill 0.4) (layers "F.Cu" "B.Cu") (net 20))
 (segment (start 147.574 75.565) (end 147.574 86.77775) (width 0.5) (layer "B.Cu") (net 20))
 (segment (start 151.638 90.805) (end 152.638 89.805) (width 0.5) (layer "B.Cu") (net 20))
 (segment (start 147.574 86.77775) (end 149.094746 88.298496) (width 0.5) (layer "B.Cu") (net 20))
 (segment (start 152.638 89.805) (end 154.178 89.805) (width 0.5) (layer "B.Cu") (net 20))
 (segment (start 148.844 83.439) (end 149.098 83.185) (width 0.5) (layer "F.Cu") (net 19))
 (segment (start 150.368 85.725) (end 150.368 78.867) (width 0.5) (layer "F.Cu") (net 19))
 (segment (start 152.4335 87.249) (end 149.098 87.249) (width 0.5) (layer "F.Cu") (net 19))
 (segment (start 150.368 78.867) (end 149.225 78.867) (width 0.5) (layer "F.Cu") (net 19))
 (segment (start 144.018 83.185) (end 144.272 83.439) (width 0.5) (layer "F.Cu") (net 19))
 (segment (start 149.098 86.995) (end 150.368 85.725) (width 0.5) (layer "F.Cu") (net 19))
 (segment (start 144.272 83.439) (end 148.844 83.439) (width 0.5) (layer "F.Cu") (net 19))
 (segment (start 149.098 87.249) (end 149.098 86.995) (width 0.5) (layer "F.Cu") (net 19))
 (via (at 152.4335 87.249) (size 0.6) (drill 0.4) (layers "F.Cu" "B.Cu") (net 19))
 (via (at 144.018 83.185) (size 0.6) (drill 0.4) (layers "F.Cu" "B.Cu") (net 19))
 (via (at 149.225 78.867) (size 0.6) (drill 0.4) (layers "F.Cu" "B.Cu") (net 19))
 (via (at 149.098 83.185) (size 0.6) (drill 0.4) (layers "F.Cu" "B.Cu") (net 19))
 (segment (start 149.098 78.994) (end 149.225 78.867) (width 0.5) (layer "B.Cu") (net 19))
 (segment (start 145.034 79.121) (end 144.018 80.137) (width 0.5) (layer "B.Cu") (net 19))
 (segment (start 149.098 83.185) (end 149.098 78.994) (width 0.5) (layer "B.Cu") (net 19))
 (segment (start 145.034 75.565) (end 145.034 79.121) (width 0.5) (layer "B.Cu") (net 19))
 (segment (start 154.178 87.265) (end 152.4495 87.265) (width 0.5) (layer "B.Cu") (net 19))
 (segment (start 144.018 80.137) (end 144.018 83.185) (width 0.5) (layer "B.Cu") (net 19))
 (segment (start 152.4495 87.265) (end 152.4335 87.249) (width 0.5) (layer "B.Cu") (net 19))
 (segment (start 154.178 87.265) (end 154.178 88.05548) (width 0.5) (layer "B.Cu") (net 19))
 (segment (start 173.007501 122.775499) (end 171.958 123.825) (width 0.5) (layer "B.Cu") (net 12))
 (segment (start 173.007501 118.841847) (end 173.007501 122.775499) (width 0.5) (layer "B.Cu") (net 12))
 (segment (start 175.497511 116.351837) (end 173.007501 118.841847) (width 0.5) (layer "B.Cu") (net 12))
 (segment (start 171.958 104.775) (end 172.228 104.775) (width 0.5) (layer "B.Cu") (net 12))
 (segment (start 175.497511 108.044511) (end 175.497511 116.351837) (width 0.5) (layer "B.Cu") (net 12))
 (segment (start 172.228 104.775) (end 175.497511 108.044511) (width 0.5) (layer "B.Cu") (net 12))
 (segment (start 161.798 116.205) (end 161.690891 116.097891) (width 0.5) (layer "F.Cu") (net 8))
 (segment (start 156.718 113.665) (end 159.150891 116.097891) (width 0.5) (layer "F.Cu") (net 8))
 (segment (start 161.798 118.745) (end 161.798 116.205) (width 0.5) (layer "F.Cu") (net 8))
 (via (at 161.690891 116.097891) (size 0.6) (drill 0.4) (layers "F.Cu" "B.Cu") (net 8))
 (via (at 159.150891 116.097891) (size 0.6) (drill 0.4) (layers "F.Cu" "B.Cu") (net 8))
 (via (at 159.150891 116.097891) (size 0.6) (drill 0.4) (layers "F.Cu" "B.Cu") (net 8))
 (via (at 156.718 113.665) (size 0.6) (drill 0.4) (layers "F.Cu" "B.Cu") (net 8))
 (via (at 161.798 118.745) (size 0.6) (drill 0.4) (layers "F.Cu" "B.Cu") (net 8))
 (segment (start 161.798 106.045) (end 156.718 111.125) (width 0.5) (layer "B.Cu") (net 8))
 (segment (start 161.798 118.745) (end 161.798 123.825) (width 0.5) (layer "B.Cu") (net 8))
 (segment (start 159.150891 116.097891) (end 159.258 116.205) (width 0.5) (layer "B.Cu") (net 8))
 (segment (start 159.150891 116.097891) (end 161.690891 116.097891) (width 0.5) (layer "B.Cu") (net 8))
 (segment (start 161.798 116.205) (end 161.690891 116.097891) (width 0.5) (layer "B.Cu") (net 8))
 (segment (start 161.798 103.505) (end 161.798 106.045) (width 0.5) (layer "B.Cu") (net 8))
 (segment (start 156.718 111.125) (end 156.718 113.665) (width 0.5) (layer "B.Cu") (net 8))
 (segment (start 171.958 118.745) (end 174.498 121.285) (width 0.5) (layer "F.Cu") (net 13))
 (via (at 171.958 118.745) (size 0.6) (drill 0.4) (layers "F.Cu" "B.Cu") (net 13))
 (via (at 174.498 121.285) (size 0.6) (drill 0.4) (layers "F.Cu" "B.Cu") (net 13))
 (segment (start 171.958 118.477826) (end 171.958 118.745) (width 0.5) (layer "B.Cu") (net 13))
 (segment (start 174.498 113.665) (end 174.498 115.937826) (width 0.5) (layer "B.Cu") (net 13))
 (segment (start 174.498 121.285) (end 174.498 123.825) (width 0.5) (layer "B.Cu") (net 13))
 (segment (start 172.228 107.315) (end 171.958 107.315) (width 0.5) (layer "B.Cu") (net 13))
 (segment (start 174.498 109.585) (end 174.498 113.665) (width 0.5) (layer "B.Cu") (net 13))
 (segment (start 172.228 107.315) (end 174.498 109.585) (width 0.5) (layer "B.Cu") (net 13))
 (segment (start 174.498 115.937826) (end 171.958 118.477826) (width 0.5) (layer "B.Cu") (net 13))
 (segment (start 147.237999 100.285001) (end 149.098 98.425) (width 0.5) (layer "B.Cu") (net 39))
 (segment (start 146.438 103.505) (end 147.237999 102.705001) (width 0.5) (layer "B.Cu") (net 39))
 (segment (start 151.638 113.665) (end 151.638 103.505) (width 0.5) (layer "B.Cu") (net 39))
 (segment (start 146.438 103.505) (end 151.638 103.505) (width 0.5) (layer "B.Cu") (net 39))
 (segment (start 149.098 98.425) (end 149.098 93.345) (width 0.5) (layer "B.Cu") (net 39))
 (segment (start 149.098 93.345) (end 147.828 92.075) (width 0.5) (layer "B.Cu") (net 39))
 (segment (start 147.237999 102.705001) (end 147.237999 100.285001) (width 0.5) (layer "B.Cu") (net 39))
 (segment (start 149.098 116.205) (end 151.638 113.665) (width 0.5) (layer "B.Cu") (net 39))
 (segment (start 146.558 116.205) (end 149.098 116.205) (width 0.5) (layer "B.Cu") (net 39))
 (segment (start 147.828 92.075) (end 145.238 92.075) (width 0.5) (layer "B.Cu") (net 39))
 (segment (start 171.958 75.565) (end 171.958 78.105) (width 0.5) (layer "B.Cu") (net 29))
 (segment (start 168.148 81.915) (end 168.148 83.185) (width 0.5) (layer "B.Cu") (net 29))
 (segment (start 171.958 78.105) (end 168.148 81.915) (width 0.5) (layer "B.Cu") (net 29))
 (segment (start 174.498 75.565) (end 174.498 78.105) (width 0.5) (layer "B.Cu") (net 30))
 (segment (start 174.498 78.105) (end 170.688 81.915) (width 0.5) (layer "B.Cu") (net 30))
 (segment (start 170.688 81.915) (end 170.688 83.185) (width 0.5) (layer "B.Cu") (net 30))
 (segment (start 123.063 84.074) (end 123.19 84.201) (width 0.5) (layer "B.Cu") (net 38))
 (segment (start 123.19 84.201) (end 125.476 84.201) (width 0.5) (layer "B.Cu") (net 38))
 (segment (start 121.158 85.979) (end 123.063 84.074) (width 0.5) (layer "B.Cu") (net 38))
 (segment (start 121.158 95.885) (end 121.158 85.979) (width 0.5) (layer "B.Cu") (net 38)))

